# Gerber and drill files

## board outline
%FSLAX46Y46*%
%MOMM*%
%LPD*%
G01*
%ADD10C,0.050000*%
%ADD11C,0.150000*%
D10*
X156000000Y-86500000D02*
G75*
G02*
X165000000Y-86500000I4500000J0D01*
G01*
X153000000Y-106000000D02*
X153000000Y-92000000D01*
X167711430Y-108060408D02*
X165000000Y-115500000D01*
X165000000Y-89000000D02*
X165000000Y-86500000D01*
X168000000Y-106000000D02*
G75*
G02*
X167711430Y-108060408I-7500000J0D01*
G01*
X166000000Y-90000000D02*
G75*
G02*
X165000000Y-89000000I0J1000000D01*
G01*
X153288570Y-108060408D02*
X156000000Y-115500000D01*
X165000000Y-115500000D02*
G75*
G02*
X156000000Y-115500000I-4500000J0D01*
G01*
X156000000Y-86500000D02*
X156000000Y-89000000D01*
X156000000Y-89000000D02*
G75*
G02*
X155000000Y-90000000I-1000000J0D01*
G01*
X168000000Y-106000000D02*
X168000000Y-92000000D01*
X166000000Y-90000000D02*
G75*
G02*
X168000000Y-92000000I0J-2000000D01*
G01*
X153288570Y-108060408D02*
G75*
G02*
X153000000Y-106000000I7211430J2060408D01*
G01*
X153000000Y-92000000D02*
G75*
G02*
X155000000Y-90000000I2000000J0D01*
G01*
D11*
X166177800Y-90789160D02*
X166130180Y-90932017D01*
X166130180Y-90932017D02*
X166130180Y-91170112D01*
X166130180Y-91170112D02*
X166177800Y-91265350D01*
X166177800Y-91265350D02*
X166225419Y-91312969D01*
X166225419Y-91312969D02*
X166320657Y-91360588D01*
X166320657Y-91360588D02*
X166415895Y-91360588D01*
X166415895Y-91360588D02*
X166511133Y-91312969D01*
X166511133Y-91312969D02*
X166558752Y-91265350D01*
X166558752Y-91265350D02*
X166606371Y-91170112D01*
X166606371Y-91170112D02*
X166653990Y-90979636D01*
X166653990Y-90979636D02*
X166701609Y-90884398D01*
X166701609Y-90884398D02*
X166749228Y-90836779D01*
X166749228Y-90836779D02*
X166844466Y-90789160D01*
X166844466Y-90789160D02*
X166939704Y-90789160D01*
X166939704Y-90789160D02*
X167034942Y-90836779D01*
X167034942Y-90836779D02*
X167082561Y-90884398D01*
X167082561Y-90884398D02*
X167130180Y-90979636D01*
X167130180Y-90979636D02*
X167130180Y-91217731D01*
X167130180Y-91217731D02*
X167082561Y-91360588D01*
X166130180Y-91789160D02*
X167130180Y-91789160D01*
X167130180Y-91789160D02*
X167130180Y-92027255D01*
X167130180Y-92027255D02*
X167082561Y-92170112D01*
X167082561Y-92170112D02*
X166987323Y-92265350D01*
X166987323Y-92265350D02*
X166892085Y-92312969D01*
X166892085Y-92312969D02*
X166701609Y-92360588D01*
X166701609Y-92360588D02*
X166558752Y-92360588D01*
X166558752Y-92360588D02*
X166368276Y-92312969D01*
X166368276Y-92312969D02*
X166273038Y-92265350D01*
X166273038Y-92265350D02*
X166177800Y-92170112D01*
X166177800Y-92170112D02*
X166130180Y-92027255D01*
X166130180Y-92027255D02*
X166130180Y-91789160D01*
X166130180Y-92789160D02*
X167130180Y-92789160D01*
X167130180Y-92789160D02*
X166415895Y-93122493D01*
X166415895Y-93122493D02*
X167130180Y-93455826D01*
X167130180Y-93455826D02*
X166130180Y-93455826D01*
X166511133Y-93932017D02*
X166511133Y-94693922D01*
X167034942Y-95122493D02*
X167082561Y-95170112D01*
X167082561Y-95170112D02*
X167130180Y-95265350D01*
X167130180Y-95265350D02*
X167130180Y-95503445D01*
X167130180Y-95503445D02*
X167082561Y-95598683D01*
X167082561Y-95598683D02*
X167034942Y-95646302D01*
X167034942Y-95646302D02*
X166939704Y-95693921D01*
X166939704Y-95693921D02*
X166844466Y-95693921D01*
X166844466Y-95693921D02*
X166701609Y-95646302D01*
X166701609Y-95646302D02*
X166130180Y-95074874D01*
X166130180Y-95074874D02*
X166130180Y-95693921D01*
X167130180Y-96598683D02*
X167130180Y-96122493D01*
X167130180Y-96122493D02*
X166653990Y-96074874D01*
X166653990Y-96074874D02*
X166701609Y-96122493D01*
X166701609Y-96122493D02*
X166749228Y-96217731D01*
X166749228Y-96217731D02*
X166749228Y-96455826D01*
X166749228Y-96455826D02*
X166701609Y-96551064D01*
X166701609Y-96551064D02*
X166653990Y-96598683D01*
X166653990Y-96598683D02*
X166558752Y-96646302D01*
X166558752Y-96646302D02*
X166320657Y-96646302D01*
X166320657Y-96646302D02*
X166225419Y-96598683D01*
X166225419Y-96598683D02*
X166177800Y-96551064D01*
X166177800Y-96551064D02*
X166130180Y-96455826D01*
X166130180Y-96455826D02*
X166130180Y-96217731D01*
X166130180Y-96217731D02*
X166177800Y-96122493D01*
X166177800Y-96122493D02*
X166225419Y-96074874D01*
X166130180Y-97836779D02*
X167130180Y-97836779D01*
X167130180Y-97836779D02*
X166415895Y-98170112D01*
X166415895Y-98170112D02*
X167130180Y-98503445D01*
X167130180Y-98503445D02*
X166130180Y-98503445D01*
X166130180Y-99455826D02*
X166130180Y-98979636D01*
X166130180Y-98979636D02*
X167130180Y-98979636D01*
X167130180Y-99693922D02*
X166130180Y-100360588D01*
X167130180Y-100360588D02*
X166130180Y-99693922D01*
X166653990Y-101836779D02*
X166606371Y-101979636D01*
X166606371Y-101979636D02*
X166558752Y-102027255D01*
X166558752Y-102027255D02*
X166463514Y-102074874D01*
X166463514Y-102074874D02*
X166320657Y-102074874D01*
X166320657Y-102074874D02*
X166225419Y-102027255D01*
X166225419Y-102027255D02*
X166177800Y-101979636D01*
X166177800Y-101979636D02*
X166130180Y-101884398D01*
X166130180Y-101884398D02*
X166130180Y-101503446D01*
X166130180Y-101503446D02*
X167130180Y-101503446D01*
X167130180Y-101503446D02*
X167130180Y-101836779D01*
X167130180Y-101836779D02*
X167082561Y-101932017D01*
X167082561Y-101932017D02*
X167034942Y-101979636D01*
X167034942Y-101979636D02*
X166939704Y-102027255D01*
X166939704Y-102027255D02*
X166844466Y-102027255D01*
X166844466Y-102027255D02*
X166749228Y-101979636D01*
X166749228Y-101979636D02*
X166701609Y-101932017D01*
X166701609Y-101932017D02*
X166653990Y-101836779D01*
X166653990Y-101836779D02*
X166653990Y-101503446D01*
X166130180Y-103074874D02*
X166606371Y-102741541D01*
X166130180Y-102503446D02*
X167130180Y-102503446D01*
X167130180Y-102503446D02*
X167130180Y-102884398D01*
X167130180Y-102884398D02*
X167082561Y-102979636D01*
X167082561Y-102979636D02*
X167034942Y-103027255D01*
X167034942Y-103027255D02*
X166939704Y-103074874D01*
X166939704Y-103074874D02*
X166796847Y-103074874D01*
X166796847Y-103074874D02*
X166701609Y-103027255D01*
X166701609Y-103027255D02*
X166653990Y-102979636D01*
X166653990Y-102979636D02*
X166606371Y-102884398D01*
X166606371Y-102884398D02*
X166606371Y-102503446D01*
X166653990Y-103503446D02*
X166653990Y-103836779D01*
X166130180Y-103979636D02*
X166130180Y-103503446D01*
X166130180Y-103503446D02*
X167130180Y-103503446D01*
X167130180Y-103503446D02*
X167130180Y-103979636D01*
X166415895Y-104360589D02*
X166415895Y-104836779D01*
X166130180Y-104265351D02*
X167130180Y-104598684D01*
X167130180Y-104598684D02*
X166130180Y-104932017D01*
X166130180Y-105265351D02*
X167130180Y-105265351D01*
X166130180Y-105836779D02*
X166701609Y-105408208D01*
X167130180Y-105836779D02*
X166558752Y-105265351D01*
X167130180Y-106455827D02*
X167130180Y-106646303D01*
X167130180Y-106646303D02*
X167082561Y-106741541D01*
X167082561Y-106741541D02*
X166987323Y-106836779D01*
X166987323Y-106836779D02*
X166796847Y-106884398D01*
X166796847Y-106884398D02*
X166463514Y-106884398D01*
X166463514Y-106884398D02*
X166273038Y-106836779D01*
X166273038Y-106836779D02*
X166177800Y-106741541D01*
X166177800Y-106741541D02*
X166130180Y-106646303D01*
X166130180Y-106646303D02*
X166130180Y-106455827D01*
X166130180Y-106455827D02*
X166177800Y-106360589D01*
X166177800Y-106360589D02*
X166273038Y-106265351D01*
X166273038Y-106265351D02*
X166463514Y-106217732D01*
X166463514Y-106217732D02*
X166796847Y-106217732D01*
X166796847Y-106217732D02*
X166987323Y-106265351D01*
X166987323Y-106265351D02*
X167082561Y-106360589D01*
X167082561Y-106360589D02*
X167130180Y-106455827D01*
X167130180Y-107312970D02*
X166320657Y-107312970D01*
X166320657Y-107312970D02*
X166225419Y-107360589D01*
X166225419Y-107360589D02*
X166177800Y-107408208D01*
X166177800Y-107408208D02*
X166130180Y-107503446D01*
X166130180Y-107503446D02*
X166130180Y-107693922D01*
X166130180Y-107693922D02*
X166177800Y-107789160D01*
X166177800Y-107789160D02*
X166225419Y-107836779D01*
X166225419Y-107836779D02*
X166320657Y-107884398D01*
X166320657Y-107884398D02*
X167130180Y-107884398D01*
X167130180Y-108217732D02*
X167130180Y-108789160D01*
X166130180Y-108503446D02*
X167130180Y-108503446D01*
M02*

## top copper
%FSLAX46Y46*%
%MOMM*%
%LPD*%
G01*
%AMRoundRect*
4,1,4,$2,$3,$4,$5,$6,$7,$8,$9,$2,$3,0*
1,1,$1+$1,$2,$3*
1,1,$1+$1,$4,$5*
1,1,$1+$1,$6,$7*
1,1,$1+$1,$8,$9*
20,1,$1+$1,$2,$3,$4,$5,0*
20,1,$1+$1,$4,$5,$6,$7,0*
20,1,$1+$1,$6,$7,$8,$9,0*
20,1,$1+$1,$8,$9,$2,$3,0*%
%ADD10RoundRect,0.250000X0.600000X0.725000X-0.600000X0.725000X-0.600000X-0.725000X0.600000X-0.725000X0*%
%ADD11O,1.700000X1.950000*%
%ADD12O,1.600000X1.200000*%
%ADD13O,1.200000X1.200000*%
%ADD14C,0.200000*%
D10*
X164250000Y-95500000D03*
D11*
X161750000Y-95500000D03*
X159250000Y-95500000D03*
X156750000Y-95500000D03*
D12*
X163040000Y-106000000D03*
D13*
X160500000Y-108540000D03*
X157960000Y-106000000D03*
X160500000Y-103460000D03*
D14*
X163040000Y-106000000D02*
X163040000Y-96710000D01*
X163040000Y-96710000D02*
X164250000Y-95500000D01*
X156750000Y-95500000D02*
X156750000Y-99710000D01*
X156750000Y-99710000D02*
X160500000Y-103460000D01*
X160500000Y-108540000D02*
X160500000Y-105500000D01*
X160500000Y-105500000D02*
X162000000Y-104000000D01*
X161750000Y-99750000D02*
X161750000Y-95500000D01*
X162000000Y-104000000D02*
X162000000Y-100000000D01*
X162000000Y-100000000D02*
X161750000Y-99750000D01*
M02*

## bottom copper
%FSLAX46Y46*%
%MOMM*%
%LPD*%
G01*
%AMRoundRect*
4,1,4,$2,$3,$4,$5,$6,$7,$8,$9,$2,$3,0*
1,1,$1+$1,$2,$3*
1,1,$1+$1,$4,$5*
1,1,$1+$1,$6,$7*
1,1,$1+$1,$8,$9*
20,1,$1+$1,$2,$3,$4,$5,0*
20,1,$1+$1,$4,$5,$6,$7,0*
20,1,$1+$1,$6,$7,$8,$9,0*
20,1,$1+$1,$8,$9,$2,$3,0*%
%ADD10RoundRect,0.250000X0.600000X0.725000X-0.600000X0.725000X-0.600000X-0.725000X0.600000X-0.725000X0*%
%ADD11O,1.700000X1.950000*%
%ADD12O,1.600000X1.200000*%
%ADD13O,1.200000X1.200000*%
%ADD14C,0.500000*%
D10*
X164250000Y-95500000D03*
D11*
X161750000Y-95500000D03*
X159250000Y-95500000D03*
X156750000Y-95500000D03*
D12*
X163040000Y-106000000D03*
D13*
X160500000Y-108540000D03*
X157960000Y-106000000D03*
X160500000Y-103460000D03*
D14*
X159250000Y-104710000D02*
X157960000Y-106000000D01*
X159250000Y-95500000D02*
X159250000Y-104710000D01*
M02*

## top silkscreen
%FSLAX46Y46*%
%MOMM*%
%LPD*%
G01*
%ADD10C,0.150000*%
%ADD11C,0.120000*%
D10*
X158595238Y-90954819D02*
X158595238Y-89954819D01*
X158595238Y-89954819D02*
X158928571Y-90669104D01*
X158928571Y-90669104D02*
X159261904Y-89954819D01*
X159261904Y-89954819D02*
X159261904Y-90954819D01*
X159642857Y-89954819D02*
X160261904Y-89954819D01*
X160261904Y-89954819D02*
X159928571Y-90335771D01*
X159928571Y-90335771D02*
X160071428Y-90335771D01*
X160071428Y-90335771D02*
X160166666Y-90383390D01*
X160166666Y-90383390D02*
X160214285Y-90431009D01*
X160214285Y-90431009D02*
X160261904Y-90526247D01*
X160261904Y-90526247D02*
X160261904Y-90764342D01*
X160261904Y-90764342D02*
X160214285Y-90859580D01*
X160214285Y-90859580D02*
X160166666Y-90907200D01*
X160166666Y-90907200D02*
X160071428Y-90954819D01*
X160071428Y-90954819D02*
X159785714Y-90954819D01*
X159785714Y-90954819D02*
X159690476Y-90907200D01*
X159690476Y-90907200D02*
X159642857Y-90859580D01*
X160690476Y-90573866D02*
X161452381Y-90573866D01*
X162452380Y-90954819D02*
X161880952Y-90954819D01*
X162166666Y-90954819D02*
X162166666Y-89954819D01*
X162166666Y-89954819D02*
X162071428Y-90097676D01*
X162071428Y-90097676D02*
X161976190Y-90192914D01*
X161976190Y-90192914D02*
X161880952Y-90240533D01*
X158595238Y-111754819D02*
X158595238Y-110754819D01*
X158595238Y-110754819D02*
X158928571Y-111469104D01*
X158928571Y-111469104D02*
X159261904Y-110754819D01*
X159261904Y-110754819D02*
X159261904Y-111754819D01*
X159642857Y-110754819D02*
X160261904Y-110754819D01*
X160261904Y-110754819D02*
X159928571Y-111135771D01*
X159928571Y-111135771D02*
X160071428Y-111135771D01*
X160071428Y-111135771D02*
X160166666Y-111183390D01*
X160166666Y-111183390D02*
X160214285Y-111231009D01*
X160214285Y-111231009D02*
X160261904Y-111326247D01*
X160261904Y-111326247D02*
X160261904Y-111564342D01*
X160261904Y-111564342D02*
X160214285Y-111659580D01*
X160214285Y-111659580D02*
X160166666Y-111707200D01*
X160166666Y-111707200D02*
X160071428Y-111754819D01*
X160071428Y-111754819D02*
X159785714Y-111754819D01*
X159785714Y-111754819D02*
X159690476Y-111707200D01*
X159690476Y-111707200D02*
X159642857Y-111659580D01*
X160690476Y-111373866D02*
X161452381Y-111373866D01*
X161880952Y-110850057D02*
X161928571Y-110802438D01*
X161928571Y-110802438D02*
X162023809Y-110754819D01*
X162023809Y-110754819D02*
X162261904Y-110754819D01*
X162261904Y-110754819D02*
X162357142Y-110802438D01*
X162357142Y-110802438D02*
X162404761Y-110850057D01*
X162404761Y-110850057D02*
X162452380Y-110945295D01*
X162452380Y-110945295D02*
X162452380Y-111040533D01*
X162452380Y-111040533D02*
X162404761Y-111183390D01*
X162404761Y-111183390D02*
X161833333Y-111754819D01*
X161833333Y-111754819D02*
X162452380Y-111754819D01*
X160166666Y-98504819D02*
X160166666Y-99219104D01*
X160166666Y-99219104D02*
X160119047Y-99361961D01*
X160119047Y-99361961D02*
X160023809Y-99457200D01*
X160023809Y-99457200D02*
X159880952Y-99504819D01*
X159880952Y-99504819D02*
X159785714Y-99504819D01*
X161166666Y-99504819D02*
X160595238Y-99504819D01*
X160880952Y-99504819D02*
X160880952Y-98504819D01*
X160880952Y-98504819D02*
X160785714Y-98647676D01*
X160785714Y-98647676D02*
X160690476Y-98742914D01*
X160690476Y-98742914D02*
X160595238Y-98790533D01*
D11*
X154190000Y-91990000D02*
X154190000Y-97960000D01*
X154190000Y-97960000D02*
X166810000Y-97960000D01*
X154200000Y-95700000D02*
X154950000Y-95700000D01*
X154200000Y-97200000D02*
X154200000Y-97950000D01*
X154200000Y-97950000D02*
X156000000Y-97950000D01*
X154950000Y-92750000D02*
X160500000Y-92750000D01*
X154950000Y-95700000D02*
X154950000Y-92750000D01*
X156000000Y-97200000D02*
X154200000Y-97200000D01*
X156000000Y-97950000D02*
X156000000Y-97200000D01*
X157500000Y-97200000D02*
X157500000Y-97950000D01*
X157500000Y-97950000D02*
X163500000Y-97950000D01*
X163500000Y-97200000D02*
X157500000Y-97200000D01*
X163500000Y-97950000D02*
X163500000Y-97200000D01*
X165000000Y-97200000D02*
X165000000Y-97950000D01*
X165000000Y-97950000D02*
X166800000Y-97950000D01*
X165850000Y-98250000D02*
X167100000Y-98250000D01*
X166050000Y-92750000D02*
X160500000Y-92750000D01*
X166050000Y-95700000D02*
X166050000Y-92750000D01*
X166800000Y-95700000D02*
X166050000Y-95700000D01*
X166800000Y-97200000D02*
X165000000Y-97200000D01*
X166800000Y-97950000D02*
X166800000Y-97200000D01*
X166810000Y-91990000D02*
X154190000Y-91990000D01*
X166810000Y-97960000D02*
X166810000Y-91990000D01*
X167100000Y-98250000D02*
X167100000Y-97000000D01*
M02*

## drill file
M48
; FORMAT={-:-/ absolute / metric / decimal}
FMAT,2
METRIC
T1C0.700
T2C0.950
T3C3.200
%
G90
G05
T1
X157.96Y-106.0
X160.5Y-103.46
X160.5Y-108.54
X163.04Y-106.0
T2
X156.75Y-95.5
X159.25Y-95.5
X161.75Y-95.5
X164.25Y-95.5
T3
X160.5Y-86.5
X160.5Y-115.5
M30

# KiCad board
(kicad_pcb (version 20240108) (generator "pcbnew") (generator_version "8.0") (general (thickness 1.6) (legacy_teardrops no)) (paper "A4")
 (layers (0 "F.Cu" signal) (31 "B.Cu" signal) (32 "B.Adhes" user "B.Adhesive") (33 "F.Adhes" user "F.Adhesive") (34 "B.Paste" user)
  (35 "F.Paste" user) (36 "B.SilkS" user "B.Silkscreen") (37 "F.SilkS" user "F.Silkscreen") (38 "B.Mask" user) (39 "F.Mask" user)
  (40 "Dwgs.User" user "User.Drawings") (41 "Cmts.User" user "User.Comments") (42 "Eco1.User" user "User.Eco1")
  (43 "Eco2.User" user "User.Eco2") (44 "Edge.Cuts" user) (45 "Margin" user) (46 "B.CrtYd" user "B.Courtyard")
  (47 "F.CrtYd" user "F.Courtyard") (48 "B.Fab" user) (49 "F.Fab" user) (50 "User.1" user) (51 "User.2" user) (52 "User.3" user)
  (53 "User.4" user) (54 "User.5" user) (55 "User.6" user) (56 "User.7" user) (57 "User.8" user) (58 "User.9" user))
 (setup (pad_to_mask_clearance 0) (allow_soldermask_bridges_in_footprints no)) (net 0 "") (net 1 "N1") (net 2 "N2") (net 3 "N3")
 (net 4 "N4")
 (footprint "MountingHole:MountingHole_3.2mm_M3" (layer "F.Cu") (at 160.5 86.5)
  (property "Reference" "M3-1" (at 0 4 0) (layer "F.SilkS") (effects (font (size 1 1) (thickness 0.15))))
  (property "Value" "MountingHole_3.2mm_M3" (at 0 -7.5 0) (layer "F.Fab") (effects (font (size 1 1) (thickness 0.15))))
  (pad "" np_thru_hole circle (at 0 0) (size 3.2 3.2) (drill 3.2) (layers "*.Cu" "*.Mask")))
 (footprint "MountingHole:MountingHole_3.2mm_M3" (layer "F.Cu") (at 160.5 115.5)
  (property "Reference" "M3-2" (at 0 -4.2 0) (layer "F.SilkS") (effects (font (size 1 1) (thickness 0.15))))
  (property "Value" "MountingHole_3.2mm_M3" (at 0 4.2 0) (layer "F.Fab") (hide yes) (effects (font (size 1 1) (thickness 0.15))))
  (pad "" np_thru_hole circle (at 0 0) (size 3.2 3.2) (drill 3.2) (layers "*.Cu" "*.Mask")))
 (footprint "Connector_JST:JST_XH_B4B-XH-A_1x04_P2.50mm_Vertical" (layer "F.Cu") (at 164.25 95.5 180)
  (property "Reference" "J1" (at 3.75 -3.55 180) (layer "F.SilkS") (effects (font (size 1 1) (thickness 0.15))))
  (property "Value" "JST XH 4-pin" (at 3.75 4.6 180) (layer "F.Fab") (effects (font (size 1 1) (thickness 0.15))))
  (fp_line (start 10.06 3.51) (end 10.06 -2.46) (stroke (width 0.12) (type solid)) (layer "F.SilkS"))
  (fp_line (start 10.06 -2.46) (end -2.56 -2.46) (stroke (width 0.12) (type solid)) (layer "F.SilkS"))
  (fp_line (start 10.05 -0.2) (end 9.3 -0.2) (stroke (width 0.12) (type solid)) (layer "F.SilkS"))
  (fp_line (start 10.05 -1.7) (end 10.05 -2.45) (stroke (width 0.12) (type solid)) (layer "F.SilkS"))
  (fp_line (start 10.05 -2.45) (end 8.25 -2.45) (stroke (width 0.12) (type solid)) (layer "F.SilkS"))
  (fp_line (start 9.3 2.75) (end 3.75 2.75) (stroke (width 0.12) (type solid)) (layer "F.SilkS"))
  (fp_line (start 9.3 -0.2) (end 9.3 2.75) (stroke (width 0.12) (type solid)) (layer "F.SilkS"))
  (fp_line (start 8.25 -1.7) (end 10.05 -1.7) (stroke (width 0.12) (type solid)) (layer "F.SilkS"))
  (fp_line (start 8.25 -2.45) (end 8.25 -1.7) (stroke (width 0.12) (type solid)) (layer "F.SilkS"))
  (fp_line (start 6.75 -1.7) (end 6.75 -2.45) (stroke (width 0.12) (type solid)) (layer "F.SilkS"))
  (fp_line (start 6.75 -2.45) (end 0.75 -2.45) (stroke (width 0.12) (type solid)) (layer "F.SilkS"))
  (fp_line (start 0.75 -1.7) (end 6.75 -1.7) (stroke (width 0.12) (type solid)) (layer "F.SilkS"))
  (fp_line (start 0.75 -2.45) (end 0.75 -1.7) (stroke (width 0.12) (type solid)) (layer "F.SilkS"))
  (fp_line (start -0.75 -1.7) (end -0.75 -2.45) (stroke (width 0.12) (type solid)) (layer "F.SilkS"))
  (fp_line (start -0.75 -2.45) (end -2.55 -2.45) (stroke (width 0.12) (type solid)) (layer "F.SilkS"))
  (fp_line (start -1.6 -2.75) (end -2.85 -2.75) (stroke (width 0.12) (type solid)) (layer "F.SilkS"))
  (fp_line (start -1.8 2.75) (end 3.75 2.75) (stroke (width 0.12) (type solid)) (layer "F.SilkS"))
  (fp_line (start -1.8 -0.2) (end -1.8 2.75) (stroke (width 0.12) (type solid)) (layer "F.SilkS"))
  (fp_line (start -2.55 -0.2) (end -1.8 -0.2) (stroke (width 0.12) (type solid)) (layer "F.SilkS"))
  (fp_line (start -2.55 -1.7) (end -0.75 -1.7) (stroke (width 0.12) (type solid)) (layer "F.SilkS"))
  (fp_line (start -2.55 -2.45) (end -2.55 -1.7) (stroke (width 0.12) (type solid)) (layer "F.SilkS"))
  (fp_line (start -2.56 3.51) (end 10.06 3.51) (stroke (width 0.12) (type solid)) (layer "F.SilkS"))
  (fp_line (start -2.56 -2.46) (end -2.56 3.51) (stroke (width 0.12) (type solid)) (layer "F.SilkS"))
  (fp_line (start -2.85 -2.75) (end -2.85 -1.5) (stroke (width 0.12) (type solid)) (layer "F.SilkS"))
  (pad "1" thru_hole roundrect (at 0 0 180) (size 1.7 1.95) (drill 0.95) (layers "*.Cu" "*.Mask") (remove_unused_layers no)
   (roundrect_rratio 0.147059) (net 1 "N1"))
  (pad "2" thru_hole oval (at 2.5 0 180) (size 1.7 1.95) (drill 0.95) (layers "*.Cu" "*.Mask") (remove_unused_layers no) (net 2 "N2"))
  (pad "3" thru_hole oval (at 5 0 180) (size 1.7 1.95) (drill 0.95) (layers "*.Cu" "*.Mask") (remove_unused_layers no) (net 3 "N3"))
  (pad "4" thru_hole oval (at 7.5 0 180) (size 1.7 1.95) (drill 0.95) (layers "*.Cu" "*.Mask") (remove_unused_layers no) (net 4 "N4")))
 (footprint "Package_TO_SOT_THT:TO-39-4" (layer "B.Cu") (at 163.04 106 180)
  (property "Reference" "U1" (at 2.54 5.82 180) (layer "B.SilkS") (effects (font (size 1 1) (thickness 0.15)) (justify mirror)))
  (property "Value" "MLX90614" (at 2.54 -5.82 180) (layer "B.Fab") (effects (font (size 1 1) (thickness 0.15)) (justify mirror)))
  (pad "1" thru_hole oval (at 0 0 180) (size 1.6 1.2) (drill 0.7) (layers "*.Cu" "*.Mask") (remove_unused_layers no) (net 1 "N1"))
  (pad "2" thru_hole oval (at 2.54 -2.54 180) (size 1.2 1.2) (drill 0.7) (layers "*.Cu" "*.Mask") (remove_unused_layers no) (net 2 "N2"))
  (pad "3" thru_hole oval (at 5.08 0 180) (size 1.2 1.2) (drill 0.7) (layers "*.Cu" "*.Mask") (remove_unused_layers no) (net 3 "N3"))
  (pad "4" thru_hole oval (at 2.54 2.54 180) (size 1.2 1.2) (drill 0.7) (layers "*.Cu" "*.Mask") (remove_unused_layers no) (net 4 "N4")))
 (gr_arc (start 156 86.5) (mid 160.5 82) (end 165 86.5) (stroke (width 0.05) (type default)) (layer "Edge.Cuts"))
 (gr_line (start 153 106) (end 153 92) (stroke (width 0.05) (type default)) (layer "Edge.Cuts"))
 (gr_line (start 167.71143 108.060408) (end 165 115.5) (stroke (width 0.05) (type default)) (layer "Edge.Cuts"))
 (gr_line (start 165 89) (end 165 86.5) (stroke (width 0.05) (type default)) (layer "Edge.Cuts"))
 (gr_arc (start 168 106) (mid 167.927507 107.040259) (end 167.71143 108.060408) (stroke (width 0.05) (type default)) (layer "Edge.Cuts"))
 (gr_arc (start 166 90) (mid 165.292893 89.707107) (end 165 89) (stroke (width 0.05) (type default)) (layer "Edge.Cuts"))
 (gr_line (start 153.28857 108.060408) (end 156 115.5) (stroke (width 0.05) (type default)) (layer "Edge.Cuts"))
 (gr_arc (start 165 115.5) (mid 160.5 120) (end 156 115.5) (stroke (width 0.05) (type default)) (layer "Edge.Cuts"))
 (gr_line (start 156 86.5) (end 156 89) (stroke (width 0.05) (type default)) (layer "Edge.Cuts"))
 (gr_arc (start 156 89) (mid 155.707107 89.707107) (end 155 90) (stroke (width 0.05) (type default)) (layer "Edge.Cuts"))
 (gr_line (start 168 106) (end 168 92) (stroke (width 0.05) (type default)) (layer "Edge.Cuts"))
 (gr_arc (start 166 90) (mid 167.414214 90.585786) (end 168 92) (stroke (width 0.05) (type default)) (layer "Edge.Cuts"))
 (gr_arc (start 153.28857 108.060408) (mid 153.072493 107.040259) (end 153 106) (stroke (width 0.05) (type default)) (layer "Edge.Cuts"))
 (gr_arc (start 153 92) (mid 153.585786 90.585786) (end 155 90) (stroke (width 0.05) (type default)) (layer "Edge.Cuts"))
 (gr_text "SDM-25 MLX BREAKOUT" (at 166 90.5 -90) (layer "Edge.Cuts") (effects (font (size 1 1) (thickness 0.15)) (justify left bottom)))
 (segment (start 163.04 106) (end 163.04 96.71) (width 0.2) (layer "F.Cu") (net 1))
 (segment (start 163.04 96.71) (end 164.25 95.5) (width 0.2) (layer "F.Cu") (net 1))
 (segment (start 156.75 95.5) (end 156.75 99.71) (width 0.2) (layer "F.Cu") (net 4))
 (segment (start 156.75 99.71) (end 160.5 103.46) (width 0.2) (layer "F.Cu") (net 4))
 (segment (start 160.5 108.54) (end 160.5 105.5) (width 0.2) (layer "F.Cu") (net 2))
 (segment (start 160.5 105.5) (end 162 104) (width 0.2) (layer "F.Cu") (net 2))
 (segment (start 161.75 99.75) (end 161.75 95.5) (width 0.2) (layer "F.Cu") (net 2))
 (segment (start 162 104) (end 162 100) (width 0.2) (layer "F.Cu") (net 2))
 (segment (start 162 100) (end 161.75 99.75) (width 0.2) (layer "F.Cu") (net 2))
 (segment (start 159.25 104.71) (end 157.96 106) (width 0.5) (layer "B.Cu") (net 3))
 (segment (start 159.25 95.5) (end 159.25 104.71) (width 0.5) (layer "B.Cu") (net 3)))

